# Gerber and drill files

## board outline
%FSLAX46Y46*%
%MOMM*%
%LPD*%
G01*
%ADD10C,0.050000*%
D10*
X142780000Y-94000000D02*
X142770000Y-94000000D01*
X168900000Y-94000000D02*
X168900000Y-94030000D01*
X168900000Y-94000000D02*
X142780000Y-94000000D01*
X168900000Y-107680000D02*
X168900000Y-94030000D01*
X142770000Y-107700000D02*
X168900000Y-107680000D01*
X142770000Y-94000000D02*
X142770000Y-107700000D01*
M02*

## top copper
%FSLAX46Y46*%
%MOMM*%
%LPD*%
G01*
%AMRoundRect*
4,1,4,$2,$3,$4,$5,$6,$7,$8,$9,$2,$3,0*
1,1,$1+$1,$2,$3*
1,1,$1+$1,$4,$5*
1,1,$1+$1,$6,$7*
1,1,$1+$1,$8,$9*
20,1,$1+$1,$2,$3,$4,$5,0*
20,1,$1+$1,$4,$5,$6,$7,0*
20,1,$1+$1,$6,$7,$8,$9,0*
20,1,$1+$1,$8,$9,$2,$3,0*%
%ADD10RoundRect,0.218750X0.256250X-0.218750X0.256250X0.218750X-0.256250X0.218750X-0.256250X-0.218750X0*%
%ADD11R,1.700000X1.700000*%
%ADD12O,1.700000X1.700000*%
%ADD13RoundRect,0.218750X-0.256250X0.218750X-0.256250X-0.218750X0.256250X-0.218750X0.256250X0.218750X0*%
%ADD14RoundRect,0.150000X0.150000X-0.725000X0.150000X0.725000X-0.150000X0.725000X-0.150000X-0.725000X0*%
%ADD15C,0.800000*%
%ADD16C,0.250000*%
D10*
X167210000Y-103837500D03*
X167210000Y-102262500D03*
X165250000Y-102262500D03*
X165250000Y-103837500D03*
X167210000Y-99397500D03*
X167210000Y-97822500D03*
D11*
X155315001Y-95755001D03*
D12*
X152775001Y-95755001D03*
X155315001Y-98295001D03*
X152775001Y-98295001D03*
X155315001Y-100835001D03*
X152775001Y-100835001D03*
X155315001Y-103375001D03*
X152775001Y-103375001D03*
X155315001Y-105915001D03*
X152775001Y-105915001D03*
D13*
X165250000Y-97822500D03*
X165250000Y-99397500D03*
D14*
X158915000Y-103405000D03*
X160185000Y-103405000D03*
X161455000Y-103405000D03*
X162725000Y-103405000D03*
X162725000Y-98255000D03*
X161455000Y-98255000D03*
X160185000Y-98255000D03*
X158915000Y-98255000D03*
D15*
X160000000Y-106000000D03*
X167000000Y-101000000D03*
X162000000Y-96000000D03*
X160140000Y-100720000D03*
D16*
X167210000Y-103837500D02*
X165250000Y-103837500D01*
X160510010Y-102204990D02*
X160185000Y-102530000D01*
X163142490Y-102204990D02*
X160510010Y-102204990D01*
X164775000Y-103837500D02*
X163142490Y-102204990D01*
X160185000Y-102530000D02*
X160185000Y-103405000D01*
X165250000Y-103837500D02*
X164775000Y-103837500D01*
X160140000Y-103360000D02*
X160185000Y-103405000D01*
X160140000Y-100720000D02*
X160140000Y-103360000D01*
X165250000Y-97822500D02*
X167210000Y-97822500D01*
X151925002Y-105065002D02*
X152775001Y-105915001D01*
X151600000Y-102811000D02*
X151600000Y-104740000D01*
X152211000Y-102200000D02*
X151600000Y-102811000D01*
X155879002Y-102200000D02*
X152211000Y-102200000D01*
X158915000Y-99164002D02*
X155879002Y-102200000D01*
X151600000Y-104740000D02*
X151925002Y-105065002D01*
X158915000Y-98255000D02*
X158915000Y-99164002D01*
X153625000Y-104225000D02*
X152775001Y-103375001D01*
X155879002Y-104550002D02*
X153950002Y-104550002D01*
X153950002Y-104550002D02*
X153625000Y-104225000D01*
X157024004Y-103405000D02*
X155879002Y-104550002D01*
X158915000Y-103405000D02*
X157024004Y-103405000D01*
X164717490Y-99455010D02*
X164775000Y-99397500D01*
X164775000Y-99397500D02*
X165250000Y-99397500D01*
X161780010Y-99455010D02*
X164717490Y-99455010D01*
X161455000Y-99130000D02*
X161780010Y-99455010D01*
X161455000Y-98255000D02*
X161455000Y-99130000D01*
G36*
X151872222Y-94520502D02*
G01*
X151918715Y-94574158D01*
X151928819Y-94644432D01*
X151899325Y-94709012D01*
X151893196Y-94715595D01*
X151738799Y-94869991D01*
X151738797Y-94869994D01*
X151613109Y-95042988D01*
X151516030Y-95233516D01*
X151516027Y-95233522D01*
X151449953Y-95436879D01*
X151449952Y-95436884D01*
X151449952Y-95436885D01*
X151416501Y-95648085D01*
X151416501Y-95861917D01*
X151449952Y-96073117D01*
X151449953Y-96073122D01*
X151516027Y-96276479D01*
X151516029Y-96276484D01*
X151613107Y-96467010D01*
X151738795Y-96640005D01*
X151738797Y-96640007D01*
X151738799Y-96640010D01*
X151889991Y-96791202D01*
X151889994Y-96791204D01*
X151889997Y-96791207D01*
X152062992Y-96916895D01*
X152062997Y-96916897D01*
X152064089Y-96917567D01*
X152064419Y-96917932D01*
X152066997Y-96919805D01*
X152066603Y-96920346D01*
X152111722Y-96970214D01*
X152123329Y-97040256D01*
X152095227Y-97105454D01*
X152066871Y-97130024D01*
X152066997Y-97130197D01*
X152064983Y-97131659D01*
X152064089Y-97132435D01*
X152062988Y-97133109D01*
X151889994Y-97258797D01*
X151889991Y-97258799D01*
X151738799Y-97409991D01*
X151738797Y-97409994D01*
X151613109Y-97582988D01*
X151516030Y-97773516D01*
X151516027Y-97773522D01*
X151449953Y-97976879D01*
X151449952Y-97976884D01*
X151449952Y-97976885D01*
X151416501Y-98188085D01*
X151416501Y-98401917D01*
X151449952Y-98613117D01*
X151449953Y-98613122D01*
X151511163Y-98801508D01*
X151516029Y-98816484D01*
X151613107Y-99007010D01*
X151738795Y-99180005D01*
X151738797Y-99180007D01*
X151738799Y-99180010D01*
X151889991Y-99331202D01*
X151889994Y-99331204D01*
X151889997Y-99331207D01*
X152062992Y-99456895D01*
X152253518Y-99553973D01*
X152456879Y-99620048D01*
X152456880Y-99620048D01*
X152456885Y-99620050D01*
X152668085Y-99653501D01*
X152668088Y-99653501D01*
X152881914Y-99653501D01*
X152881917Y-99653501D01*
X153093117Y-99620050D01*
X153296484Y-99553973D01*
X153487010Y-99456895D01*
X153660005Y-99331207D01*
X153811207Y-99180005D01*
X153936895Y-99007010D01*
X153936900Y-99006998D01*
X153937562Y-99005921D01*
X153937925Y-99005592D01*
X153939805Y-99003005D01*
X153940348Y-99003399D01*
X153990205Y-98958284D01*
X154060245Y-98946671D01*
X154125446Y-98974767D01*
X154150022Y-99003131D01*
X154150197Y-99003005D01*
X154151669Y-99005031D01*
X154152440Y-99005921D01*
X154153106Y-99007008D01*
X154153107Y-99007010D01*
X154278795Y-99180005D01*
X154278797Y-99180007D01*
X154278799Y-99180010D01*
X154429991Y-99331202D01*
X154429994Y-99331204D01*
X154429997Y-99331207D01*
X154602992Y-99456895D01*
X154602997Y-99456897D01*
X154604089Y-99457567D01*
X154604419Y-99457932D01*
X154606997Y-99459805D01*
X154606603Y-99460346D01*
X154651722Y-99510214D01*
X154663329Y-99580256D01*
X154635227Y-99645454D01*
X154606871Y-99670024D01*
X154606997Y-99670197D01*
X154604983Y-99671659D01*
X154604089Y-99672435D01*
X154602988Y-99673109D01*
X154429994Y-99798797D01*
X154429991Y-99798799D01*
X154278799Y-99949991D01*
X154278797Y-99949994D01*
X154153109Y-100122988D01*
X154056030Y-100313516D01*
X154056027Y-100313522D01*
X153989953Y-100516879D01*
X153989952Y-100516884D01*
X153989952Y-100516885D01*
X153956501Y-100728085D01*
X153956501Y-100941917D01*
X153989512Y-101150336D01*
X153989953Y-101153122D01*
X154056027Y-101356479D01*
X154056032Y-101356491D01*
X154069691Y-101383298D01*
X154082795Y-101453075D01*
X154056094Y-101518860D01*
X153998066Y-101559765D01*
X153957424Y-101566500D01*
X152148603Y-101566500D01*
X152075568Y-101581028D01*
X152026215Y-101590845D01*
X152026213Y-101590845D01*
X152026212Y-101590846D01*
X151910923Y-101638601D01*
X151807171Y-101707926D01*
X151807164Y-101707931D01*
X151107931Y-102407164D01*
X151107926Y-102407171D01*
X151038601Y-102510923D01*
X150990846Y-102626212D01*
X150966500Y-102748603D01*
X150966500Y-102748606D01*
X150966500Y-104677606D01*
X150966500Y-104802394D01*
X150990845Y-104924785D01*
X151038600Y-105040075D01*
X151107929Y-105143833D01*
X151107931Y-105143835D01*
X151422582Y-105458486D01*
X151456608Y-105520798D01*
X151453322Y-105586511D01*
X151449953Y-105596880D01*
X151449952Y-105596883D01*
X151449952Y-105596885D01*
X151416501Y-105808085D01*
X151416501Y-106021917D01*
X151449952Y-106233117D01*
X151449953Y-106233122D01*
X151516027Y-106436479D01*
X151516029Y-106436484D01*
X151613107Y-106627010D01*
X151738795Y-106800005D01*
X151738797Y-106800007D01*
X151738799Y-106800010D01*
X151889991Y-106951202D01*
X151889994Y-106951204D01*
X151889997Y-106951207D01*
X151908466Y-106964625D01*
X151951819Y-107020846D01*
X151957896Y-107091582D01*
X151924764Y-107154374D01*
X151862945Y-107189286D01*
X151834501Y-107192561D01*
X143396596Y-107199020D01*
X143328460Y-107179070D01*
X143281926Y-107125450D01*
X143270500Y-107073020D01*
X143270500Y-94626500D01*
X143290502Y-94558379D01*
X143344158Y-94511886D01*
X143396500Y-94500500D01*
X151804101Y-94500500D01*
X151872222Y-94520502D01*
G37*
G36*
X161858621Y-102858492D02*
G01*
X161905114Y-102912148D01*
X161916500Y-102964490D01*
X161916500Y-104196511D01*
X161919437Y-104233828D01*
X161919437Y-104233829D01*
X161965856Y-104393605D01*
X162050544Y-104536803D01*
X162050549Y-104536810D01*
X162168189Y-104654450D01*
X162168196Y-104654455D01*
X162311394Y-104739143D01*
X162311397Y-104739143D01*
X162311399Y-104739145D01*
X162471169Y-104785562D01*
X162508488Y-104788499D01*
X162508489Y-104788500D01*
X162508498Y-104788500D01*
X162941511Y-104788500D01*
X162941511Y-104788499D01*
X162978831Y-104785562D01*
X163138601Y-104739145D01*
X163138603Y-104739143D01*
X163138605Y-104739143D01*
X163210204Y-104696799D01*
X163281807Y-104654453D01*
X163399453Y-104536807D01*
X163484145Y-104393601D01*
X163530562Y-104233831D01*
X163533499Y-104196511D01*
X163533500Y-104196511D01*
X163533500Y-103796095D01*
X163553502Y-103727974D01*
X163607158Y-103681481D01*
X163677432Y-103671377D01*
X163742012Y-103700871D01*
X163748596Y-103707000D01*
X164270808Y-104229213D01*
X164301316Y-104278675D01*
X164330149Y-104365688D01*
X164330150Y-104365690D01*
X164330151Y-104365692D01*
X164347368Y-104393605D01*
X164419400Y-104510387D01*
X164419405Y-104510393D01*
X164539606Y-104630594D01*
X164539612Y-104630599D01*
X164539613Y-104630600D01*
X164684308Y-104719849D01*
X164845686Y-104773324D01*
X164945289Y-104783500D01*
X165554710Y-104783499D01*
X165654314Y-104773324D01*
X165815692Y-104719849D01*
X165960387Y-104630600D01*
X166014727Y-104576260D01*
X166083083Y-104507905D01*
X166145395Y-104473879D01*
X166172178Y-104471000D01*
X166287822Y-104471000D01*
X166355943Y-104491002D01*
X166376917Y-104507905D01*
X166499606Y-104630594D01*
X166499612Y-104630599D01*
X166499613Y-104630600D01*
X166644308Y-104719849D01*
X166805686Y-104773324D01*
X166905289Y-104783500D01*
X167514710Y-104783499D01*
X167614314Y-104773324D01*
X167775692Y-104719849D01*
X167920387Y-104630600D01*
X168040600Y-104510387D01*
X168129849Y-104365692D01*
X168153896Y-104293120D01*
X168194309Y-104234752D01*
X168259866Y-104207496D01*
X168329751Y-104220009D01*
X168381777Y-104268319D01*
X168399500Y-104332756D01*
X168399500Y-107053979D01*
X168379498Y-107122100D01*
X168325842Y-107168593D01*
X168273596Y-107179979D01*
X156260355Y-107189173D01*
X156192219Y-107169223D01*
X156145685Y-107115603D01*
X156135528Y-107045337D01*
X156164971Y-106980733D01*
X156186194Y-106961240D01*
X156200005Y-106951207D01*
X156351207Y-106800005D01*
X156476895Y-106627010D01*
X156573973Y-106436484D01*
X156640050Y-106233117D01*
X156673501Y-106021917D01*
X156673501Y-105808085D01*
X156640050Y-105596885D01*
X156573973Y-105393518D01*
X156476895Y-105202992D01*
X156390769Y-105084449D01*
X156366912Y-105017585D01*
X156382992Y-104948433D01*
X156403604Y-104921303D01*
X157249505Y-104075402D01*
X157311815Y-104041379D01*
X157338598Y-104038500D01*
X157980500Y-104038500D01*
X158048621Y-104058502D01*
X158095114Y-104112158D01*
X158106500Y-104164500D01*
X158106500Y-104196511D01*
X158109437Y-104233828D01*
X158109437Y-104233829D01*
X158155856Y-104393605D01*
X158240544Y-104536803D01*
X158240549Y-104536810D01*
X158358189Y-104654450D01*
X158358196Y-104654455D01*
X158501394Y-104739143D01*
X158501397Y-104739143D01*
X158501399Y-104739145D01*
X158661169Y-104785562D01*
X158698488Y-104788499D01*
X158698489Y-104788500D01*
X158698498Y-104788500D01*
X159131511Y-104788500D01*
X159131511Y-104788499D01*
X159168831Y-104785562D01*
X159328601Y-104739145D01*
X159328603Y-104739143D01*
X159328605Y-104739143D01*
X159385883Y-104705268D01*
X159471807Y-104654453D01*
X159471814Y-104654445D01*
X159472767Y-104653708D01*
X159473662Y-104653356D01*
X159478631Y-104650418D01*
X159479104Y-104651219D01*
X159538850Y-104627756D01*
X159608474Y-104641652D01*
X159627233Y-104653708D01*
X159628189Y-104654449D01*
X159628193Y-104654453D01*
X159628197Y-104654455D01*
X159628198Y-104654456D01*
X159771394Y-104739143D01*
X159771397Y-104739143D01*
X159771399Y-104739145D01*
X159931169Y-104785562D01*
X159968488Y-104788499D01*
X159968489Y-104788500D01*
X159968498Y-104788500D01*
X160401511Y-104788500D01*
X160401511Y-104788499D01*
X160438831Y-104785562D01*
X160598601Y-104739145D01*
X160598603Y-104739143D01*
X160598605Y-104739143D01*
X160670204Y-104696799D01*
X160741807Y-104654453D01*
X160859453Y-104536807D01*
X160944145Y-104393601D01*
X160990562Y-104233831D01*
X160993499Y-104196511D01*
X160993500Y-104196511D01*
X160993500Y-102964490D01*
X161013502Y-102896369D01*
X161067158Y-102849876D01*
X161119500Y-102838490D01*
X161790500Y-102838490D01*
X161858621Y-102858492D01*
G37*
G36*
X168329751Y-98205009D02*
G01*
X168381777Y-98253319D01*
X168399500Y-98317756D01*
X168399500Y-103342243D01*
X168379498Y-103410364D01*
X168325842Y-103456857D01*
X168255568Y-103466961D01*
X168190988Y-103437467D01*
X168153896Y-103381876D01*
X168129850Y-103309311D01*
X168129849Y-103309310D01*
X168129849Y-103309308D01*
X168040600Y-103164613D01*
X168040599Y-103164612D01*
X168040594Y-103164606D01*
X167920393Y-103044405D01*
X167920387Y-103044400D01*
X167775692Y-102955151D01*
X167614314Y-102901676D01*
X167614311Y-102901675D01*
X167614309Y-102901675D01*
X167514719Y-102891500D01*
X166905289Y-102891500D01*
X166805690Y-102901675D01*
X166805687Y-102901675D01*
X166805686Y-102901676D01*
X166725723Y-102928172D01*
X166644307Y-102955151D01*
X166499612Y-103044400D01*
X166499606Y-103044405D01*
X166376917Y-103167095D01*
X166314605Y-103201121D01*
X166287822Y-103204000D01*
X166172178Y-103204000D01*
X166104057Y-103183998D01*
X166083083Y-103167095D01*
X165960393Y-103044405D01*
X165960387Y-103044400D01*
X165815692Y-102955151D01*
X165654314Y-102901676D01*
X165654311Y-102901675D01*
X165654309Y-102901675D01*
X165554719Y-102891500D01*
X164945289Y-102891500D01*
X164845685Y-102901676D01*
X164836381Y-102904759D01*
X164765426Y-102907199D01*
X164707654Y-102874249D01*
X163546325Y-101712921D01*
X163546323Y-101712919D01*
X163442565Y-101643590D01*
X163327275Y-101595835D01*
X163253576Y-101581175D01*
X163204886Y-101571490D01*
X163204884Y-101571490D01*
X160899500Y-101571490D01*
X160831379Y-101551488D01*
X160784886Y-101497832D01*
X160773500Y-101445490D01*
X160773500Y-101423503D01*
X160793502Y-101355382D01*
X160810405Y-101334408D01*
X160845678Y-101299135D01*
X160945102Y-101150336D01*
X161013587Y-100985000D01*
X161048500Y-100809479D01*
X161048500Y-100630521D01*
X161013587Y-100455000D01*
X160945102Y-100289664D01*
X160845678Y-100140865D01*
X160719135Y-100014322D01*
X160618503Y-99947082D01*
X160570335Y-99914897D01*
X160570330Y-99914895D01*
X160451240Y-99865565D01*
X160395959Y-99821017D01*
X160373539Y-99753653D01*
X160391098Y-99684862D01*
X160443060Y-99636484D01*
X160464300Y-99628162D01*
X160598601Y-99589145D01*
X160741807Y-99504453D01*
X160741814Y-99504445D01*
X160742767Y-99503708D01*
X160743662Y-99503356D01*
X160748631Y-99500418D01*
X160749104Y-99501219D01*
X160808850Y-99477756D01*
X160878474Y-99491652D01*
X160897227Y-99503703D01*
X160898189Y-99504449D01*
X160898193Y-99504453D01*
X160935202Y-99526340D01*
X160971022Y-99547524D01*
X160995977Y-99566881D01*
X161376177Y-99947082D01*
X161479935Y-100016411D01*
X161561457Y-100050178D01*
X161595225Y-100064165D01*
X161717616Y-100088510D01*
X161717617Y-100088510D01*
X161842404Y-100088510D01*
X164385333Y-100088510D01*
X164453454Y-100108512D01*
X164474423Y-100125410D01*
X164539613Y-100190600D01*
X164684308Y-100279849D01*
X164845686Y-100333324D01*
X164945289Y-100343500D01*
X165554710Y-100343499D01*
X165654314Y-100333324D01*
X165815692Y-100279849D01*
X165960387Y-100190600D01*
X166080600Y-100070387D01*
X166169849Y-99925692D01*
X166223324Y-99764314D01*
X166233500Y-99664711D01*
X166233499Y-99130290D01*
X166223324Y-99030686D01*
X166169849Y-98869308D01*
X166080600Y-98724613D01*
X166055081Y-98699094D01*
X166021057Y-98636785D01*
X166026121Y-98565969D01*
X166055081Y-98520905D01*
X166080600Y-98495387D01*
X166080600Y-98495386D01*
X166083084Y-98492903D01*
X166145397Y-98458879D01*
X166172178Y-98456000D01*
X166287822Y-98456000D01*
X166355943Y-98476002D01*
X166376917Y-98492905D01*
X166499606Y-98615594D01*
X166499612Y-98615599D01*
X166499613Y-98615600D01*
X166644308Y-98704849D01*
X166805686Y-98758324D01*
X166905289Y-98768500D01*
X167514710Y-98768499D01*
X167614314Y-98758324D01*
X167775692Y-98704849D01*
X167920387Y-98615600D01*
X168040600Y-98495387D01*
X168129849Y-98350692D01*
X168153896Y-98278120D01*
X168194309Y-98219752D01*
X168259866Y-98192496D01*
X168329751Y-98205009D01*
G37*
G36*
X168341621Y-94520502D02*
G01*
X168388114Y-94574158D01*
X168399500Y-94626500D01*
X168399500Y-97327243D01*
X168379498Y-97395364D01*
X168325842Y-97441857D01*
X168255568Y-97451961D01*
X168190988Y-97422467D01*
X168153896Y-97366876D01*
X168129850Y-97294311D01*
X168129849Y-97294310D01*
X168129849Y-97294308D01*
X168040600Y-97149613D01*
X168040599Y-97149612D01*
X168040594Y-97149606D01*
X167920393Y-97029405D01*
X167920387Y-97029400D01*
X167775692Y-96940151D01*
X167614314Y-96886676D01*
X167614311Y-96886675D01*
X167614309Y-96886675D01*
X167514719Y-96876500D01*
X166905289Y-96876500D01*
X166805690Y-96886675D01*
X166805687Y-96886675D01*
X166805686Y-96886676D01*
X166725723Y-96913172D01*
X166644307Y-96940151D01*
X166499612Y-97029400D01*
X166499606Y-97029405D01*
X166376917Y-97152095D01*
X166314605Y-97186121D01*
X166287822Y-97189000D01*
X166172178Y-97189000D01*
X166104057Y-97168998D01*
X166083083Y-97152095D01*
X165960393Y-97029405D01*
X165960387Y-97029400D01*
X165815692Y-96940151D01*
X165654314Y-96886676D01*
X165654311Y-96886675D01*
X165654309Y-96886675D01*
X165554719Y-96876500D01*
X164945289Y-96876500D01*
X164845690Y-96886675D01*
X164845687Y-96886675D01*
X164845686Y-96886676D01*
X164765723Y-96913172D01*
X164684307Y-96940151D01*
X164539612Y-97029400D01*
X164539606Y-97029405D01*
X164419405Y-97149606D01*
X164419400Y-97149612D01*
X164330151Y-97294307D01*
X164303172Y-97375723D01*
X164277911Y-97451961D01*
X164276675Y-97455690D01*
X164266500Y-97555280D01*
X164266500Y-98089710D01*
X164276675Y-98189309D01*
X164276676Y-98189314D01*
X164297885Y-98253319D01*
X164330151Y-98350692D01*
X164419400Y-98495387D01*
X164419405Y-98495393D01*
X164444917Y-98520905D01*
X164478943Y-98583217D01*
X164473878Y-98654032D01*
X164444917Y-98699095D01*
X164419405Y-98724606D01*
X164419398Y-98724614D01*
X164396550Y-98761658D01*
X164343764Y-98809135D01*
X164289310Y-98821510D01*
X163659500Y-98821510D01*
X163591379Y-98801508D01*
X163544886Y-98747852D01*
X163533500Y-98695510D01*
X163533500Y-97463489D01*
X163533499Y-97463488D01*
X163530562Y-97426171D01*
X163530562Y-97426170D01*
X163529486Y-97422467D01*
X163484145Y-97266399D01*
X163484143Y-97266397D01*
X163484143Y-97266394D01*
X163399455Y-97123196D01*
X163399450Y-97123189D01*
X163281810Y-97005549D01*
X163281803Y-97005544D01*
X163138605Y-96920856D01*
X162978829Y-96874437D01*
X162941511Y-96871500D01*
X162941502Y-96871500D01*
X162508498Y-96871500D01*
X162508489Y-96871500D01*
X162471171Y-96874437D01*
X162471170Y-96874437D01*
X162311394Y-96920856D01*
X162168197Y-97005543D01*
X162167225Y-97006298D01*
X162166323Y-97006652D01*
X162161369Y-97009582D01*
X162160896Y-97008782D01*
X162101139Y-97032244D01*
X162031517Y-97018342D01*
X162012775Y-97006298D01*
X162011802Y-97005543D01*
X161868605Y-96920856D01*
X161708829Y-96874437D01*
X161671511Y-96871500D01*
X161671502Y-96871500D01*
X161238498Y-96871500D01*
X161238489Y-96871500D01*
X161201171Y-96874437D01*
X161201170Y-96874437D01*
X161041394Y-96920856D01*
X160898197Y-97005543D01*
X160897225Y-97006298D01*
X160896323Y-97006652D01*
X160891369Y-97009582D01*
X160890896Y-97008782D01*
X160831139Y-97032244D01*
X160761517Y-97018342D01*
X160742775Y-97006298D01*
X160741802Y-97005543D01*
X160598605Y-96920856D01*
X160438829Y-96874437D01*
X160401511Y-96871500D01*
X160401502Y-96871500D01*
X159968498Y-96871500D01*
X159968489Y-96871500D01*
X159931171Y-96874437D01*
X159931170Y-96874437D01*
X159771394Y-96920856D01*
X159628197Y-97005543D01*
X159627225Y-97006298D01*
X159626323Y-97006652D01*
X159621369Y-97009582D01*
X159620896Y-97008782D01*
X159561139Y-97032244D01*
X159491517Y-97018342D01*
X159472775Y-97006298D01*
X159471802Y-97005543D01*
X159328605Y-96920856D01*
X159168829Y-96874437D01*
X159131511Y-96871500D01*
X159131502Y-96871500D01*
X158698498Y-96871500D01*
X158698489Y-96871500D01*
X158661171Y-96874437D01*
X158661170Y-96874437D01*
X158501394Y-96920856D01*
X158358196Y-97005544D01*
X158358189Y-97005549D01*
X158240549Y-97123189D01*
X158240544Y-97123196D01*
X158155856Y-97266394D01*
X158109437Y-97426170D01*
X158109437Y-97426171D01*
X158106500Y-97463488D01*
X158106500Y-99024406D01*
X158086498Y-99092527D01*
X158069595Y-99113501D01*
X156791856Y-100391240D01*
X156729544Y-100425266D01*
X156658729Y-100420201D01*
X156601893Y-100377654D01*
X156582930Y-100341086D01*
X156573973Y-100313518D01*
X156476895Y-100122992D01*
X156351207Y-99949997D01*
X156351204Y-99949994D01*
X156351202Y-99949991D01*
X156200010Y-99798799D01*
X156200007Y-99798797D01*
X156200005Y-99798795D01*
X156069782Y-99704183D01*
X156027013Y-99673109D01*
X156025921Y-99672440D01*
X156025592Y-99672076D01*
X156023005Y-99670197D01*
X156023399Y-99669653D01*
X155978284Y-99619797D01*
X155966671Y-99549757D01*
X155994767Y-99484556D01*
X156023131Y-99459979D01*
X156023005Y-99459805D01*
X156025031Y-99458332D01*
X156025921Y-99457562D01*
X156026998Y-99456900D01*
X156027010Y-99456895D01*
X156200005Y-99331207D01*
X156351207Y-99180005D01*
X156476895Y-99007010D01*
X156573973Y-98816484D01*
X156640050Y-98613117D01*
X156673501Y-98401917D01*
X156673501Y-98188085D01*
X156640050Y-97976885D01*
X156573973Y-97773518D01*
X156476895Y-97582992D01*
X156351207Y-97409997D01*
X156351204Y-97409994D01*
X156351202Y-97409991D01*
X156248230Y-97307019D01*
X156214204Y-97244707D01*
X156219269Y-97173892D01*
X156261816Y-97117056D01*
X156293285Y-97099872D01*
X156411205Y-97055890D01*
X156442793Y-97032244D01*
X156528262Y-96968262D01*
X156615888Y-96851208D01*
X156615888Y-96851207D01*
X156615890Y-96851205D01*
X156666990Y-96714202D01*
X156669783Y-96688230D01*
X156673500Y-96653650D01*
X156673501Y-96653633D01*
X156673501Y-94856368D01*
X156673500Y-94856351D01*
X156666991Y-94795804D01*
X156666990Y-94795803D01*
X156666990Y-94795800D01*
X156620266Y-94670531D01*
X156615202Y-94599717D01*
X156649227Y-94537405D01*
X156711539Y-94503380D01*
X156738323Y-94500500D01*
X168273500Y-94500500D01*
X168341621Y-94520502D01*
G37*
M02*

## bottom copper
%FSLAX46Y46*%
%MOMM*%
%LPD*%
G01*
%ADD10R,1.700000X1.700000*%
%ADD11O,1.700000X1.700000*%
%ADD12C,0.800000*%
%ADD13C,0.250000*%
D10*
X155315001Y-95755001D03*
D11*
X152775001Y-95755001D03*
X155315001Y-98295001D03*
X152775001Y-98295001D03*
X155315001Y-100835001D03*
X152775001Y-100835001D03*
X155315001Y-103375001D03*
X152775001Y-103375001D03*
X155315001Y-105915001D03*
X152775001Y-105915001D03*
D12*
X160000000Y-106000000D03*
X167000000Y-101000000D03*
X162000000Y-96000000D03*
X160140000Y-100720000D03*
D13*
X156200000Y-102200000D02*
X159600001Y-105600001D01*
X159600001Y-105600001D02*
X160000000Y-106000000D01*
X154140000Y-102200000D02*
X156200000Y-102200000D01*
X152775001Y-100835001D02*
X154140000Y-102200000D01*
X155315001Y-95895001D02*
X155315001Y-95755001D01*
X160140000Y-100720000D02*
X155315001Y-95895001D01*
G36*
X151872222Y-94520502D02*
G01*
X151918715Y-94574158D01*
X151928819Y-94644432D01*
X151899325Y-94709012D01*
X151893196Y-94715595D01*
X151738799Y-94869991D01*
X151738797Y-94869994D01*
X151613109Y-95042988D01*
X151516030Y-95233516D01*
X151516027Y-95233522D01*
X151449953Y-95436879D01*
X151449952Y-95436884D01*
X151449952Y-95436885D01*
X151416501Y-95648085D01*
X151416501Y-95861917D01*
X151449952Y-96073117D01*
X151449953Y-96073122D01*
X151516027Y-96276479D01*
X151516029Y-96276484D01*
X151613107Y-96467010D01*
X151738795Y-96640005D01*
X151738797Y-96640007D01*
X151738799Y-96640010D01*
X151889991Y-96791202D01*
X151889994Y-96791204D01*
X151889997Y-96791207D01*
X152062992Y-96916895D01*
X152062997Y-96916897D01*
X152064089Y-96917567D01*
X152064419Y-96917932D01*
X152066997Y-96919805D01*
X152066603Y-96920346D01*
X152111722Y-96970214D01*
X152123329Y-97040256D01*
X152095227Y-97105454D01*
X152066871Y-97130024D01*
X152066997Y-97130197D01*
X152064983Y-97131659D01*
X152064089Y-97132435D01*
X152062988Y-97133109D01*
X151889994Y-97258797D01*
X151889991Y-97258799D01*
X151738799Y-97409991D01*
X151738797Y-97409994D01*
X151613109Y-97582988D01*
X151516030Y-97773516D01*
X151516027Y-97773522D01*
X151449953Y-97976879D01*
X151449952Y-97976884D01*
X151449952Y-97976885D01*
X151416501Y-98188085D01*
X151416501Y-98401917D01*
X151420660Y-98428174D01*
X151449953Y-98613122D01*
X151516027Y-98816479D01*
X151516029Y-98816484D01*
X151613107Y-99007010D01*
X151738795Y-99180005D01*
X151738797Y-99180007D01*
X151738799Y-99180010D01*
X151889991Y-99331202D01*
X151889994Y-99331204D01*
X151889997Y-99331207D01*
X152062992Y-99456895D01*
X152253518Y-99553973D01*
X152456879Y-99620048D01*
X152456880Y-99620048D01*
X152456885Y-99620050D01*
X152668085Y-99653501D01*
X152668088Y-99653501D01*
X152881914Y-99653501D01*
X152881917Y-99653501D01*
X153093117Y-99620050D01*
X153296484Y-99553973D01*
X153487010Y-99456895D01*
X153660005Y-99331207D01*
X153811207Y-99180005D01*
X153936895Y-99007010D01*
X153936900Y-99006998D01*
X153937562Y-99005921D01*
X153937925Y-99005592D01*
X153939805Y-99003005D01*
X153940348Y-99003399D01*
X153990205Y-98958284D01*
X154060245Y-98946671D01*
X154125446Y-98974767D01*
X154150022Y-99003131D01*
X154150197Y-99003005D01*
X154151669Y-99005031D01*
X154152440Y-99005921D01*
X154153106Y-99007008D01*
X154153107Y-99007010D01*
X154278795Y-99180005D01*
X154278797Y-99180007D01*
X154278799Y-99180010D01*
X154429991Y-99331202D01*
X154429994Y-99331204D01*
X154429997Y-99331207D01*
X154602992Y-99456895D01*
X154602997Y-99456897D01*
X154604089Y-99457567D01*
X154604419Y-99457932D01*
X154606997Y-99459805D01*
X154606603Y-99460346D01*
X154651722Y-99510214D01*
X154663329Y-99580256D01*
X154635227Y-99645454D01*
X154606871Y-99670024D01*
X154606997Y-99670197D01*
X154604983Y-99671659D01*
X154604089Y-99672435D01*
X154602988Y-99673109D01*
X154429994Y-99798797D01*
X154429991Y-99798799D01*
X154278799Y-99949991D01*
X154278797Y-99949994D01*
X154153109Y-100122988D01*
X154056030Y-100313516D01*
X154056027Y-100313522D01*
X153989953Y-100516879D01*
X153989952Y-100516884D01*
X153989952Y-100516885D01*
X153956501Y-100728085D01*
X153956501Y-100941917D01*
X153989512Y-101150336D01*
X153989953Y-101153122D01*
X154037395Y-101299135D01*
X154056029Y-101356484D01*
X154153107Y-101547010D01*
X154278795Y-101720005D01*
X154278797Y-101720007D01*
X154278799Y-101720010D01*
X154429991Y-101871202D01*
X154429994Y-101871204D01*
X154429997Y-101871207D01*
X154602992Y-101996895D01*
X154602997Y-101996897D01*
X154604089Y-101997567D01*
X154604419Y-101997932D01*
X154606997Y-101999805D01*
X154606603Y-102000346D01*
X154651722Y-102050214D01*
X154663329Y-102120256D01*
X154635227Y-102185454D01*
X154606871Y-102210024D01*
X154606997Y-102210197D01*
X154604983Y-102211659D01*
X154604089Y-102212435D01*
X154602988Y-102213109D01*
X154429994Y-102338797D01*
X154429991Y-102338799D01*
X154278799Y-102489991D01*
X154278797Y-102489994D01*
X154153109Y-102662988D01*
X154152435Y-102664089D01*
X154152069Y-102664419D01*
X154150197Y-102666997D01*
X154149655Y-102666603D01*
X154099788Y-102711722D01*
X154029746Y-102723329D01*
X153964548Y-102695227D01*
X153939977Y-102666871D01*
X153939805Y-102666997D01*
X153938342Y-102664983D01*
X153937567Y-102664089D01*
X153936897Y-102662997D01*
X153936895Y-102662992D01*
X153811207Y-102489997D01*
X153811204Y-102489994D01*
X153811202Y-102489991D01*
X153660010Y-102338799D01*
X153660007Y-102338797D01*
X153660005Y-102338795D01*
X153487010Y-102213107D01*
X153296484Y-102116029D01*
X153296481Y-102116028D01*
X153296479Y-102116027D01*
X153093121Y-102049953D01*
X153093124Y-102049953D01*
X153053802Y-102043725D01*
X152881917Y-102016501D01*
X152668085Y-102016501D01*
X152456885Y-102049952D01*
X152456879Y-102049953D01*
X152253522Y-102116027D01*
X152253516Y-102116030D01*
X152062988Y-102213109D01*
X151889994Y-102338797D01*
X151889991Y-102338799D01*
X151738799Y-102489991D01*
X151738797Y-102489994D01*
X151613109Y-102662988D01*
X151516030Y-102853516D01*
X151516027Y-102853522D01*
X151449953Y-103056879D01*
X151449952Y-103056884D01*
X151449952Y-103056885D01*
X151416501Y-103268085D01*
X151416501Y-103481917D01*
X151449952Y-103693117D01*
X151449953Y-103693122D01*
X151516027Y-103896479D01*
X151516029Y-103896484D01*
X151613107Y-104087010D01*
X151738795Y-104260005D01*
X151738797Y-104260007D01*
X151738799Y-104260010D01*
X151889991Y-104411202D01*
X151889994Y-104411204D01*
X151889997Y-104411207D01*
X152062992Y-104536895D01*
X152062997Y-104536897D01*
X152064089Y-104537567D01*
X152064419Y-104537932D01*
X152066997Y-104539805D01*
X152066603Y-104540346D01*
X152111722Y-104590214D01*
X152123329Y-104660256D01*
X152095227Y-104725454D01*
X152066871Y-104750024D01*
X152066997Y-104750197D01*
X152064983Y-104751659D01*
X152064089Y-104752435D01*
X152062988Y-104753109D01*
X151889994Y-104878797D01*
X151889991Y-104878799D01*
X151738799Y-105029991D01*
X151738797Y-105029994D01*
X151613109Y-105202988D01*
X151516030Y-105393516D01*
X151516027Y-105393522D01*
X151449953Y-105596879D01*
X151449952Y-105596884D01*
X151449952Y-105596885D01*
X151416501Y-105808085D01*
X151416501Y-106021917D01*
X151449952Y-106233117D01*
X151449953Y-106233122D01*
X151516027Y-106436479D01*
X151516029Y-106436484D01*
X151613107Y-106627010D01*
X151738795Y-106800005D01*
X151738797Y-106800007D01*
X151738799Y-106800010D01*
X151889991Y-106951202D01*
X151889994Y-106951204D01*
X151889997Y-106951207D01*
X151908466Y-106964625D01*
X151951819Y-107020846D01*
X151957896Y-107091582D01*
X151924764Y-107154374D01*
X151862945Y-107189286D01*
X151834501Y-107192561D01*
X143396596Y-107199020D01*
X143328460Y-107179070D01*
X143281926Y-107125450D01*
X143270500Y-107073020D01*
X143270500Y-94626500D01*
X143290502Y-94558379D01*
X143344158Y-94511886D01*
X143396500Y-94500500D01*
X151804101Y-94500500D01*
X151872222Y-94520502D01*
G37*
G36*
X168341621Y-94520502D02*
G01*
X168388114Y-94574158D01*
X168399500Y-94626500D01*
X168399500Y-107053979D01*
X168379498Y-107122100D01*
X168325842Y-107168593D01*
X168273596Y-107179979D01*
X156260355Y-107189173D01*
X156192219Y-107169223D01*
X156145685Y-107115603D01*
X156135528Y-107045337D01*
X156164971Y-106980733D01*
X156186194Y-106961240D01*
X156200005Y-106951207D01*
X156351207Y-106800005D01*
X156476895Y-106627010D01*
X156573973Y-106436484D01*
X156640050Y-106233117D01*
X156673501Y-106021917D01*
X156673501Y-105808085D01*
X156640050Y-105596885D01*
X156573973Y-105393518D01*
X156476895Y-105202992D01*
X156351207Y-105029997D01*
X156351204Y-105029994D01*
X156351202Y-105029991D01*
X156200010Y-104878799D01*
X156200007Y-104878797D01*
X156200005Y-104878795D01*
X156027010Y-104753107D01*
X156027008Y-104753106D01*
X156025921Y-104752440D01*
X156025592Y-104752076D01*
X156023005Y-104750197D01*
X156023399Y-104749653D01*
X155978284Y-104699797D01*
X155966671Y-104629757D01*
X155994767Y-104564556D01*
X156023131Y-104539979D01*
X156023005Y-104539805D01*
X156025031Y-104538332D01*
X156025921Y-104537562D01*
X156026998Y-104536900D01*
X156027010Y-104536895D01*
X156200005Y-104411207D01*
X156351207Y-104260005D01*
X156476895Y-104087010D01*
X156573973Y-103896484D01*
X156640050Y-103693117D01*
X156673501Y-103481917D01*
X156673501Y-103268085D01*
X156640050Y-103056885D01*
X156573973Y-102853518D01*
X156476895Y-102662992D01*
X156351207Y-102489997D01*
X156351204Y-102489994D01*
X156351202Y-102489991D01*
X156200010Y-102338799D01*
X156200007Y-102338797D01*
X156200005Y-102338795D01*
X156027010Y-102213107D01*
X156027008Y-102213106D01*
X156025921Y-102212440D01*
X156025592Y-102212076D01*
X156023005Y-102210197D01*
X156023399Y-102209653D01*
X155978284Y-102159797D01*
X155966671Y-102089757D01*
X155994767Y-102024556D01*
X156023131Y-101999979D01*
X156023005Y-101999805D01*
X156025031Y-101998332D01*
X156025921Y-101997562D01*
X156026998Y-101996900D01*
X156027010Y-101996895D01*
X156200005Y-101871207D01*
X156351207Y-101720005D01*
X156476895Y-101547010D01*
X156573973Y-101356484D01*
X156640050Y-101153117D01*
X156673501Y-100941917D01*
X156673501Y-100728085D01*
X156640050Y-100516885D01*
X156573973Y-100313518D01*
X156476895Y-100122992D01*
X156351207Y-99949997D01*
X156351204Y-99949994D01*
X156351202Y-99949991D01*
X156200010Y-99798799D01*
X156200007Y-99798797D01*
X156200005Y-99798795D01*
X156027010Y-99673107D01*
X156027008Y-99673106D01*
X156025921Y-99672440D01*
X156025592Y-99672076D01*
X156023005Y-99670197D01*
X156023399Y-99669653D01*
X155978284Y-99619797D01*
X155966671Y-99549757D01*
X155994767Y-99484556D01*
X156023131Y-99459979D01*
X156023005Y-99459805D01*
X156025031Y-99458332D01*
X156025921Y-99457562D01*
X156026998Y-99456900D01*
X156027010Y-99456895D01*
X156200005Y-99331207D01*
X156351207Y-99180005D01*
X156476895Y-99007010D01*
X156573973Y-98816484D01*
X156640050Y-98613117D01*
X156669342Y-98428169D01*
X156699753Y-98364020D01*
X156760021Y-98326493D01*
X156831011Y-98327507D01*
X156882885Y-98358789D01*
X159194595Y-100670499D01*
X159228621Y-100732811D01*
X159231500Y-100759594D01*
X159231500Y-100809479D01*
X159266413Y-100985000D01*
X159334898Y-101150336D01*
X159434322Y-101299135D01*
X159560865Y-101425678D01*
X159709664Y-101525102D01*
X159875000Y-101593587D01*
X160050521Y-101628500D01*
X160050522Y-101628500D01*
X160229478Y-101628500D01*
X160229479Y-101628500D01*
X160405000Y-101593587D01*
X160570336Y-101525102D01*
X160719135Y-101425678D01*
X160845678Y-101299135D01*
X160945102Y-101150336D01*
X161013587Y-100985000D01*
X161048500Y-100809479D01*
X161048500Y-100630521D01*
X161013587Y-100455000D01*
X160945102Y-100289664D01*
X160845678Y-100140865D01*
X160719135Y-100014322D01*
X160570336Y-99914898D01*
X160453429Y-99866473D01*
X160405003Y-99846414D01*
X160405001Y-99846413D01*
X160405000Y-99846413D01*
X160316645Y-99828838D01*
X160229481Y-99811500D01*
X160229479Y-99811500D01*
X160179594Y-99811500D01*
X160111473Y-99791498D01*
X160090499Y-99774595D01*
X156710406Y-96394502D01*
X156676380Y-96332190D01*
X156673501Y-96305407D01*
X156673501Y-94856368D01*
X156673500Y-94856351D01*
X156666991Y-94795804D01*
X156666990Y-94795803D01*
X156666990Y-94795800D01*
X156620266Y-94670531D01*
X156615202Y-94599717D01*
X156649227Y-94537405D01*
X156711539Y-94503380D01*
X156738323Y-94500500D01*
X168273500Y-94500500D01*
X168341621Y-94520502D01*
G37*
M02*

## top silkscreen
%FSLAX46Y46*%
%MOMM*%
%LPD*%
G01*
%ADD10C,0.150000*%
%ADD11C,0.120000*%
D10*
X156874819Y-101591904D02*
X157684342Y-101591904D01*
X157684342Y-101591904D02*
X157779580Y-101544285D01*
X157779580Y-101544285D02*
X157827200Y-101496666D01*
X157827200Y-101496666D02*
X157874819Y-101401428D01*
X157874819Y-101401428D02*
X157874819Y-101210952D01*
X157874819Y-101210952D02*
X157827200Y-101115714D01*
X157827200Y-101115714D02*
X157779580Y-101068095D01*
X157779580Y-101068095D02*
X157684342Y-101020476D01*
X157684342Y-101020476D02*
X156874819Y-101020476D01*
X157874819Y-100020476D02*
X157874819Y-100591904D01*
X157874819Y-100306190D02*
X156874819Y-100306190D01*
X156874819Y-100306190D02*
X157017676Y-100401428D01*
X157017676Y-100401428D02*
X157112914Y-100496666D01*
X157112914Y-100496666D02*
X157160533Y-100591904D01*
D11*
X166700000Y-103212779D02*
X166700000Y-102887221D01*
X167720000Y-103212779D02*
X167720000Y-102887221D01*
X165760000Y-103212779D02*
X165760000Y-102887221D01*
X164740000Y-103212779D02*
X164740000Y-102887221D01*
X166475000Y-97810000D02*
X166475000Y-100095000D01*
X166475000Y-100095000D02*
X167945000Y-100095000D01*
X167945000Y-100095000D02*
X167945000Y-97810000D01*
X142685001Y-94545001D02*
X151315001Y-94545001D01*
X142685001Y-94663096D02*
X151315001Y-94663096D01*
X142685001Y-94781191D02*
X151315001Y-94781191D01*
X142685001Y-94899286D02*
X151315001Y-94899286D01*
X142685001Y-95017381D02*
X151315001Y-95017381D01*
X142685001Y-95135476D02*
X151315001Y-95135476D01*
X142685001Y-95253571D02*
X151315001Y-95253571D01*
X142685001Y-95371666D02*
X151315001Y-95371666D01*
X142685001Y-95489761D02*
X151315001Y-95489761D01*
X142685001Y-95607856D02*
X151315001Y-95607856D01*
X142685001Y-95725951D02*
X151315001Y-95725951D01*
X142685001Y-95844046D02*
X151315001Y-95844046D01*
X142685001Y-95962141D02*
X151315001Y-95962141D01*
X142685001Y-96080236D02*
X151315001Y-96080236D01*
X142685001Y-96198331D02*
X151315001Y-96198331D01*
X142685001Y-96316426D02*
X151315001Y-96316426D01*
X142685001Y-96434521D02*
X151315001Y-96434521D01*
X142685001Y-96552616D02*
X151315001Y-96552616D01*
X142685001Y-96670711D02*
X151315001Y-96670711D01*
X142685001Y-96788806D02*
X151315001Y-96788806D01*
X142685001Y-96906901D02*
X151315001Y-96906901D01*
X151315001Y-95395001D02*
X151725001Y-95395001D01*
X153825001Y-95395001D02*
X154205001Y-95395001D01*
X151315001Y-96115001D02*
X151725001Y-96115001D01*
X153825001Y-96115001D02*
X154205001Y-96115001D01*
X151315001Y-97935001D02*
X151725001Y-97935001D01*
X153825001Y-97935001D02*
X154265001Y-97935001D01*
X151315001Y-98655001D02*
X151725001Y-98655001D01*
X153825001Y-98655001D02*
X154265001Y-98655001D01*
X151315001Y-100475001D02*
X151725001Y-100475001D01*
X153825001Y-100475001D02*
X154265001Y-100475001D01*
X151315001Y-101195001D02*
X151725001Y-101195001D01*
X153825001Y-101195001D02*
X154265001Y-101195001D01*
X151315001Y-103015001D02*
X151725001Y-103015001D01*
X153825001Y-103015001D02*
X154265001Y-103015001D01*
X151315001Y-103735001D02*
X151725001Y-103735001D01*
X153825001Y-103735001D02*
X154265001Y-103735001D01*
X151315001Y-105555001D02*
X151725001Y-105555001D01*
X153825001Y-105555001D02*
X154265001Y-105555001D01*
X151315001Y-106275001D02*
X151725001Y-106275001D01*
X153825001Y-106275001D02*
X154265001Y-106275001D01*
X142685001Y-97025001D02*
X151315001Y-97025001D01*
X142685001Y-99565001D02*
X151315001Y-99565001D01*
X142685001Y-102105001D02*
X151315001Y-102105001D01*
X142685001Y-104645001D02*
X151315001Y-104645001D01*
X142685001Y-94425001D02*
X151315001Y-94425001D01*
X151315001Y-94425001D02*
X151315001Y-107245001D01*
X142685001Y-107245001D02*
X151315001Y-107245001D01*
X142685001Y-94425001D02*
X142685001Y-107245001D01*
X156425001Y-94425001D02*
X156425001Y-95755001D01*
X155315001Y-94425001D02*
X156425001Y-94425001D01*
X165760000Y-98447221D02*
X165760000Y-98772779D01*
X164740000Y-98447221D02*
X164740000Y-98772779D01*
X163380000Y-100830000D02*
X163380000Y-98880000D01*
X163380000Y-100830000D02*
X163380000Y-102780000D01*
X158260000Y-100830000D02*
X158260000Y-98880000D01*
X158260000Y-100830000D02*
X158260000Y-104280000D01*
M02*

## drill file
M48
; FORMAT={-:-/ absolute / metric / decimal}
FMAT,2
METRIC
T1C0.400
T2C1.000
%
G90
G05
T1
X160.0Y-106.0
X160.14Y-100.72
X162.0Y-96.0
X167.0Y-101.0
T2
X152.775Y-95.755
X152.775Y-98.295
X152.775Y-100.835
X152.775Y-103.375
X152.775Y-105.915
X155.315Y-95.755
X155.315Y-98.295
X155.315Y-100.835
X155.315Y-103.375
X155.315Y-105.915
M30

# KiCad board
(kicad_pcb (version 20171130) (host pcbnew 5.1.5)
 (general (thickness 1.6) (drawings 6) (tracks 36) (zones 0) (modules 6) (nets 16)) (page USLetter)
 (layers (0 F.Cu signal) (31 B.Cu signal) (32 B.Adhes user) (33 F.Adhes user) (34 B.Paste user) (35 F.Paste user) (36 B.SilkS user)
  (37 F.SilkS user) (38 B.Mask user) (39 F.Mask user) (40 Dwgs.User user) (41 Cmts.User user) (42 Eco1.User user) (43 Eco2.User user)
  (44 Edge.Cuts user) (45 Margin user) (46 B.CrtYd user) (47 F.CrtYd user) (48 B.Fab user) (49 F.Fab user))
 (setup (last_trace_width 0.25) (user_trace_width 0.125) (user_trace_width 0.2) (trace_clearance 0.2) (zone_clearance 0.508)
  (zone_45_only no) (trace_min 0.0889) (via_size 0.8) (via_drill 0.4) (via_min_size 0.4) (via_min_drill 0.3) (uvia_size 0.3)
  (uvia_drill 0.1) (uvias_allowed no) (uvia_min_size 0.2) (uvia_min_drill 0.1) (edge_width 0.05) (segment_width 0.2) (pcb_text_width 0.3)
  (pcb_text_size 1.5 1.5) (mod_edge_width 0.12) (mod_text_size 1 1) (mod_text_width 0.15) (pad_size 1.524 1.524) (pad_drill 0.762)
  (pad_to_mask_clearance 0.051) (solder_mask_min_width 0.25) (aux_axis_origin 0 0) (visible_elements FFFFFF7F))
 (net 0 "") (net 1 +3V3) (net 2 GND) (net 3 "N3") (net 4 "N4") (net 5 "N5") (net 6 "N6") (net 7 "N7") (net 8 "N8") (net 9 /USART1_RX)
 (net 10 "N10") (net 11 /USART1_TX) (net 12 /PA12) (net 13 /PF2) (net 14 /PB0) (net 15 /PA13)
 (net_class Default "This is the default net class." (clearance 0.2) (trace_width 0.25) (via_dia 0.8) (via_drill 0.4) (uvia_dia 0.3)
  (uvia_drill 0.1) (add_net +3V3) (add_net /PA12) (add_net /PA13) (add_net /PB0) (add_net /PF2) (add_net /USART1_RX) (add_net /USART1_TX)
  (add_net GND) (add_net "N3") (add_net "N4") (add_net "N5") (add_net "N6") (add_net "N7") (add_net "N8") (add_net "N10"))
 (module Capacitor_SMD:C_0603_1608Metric (layer F.Cu) (at 167.21 103.05 90)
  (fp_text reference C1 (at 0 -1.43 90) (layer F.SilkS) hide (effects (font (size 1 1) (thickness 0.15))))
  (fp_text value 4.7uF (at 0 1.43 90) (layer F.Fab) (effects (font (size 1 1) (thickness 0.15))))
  (fp_line (start -0.162779 -0.51) (end 0.162779 -0.51) (layer F.SilkS) (width 0.12))
  (fp_line (start -0.162779 0.51) (end 0.162779 0.51) (layer F.SilkS) (width 0.12))
  (pad 1 smd roundrect (at -0.7875 0 90) (size 0.875 0.95) (layers F.Cu F.Paste F.Mask) (roundrect_rratio 0.25) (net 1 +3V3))
  (pad 2 smd roundrect (at 0.7875 0 90) (size 0.875 0.95) (layers F.Cu F.Paste F.Mask) (roundrect_rratio 0.25) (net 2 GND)))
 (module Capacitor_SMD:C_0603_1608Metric (layer F.Cu) (at 165.25 103.05 90)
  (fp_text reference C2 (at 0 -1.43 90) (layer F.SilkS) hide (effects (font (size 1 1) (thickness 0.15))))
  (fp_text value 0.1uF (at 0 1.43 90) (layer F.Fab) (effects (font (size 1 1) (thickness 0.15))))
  (fp_line (start -0.162779 0.51) (end 0.162779 0.51) (layer F.SilkS) (width 0.12))
  (fp_line (start -0.162779 -0.51) (end 0.162779 -0.51) (layer F.SilkS) (width 0.12))
  (pad 2 smd roundrect (at 0.7875 0 90) (size 0.875 0.95) (layers F.Cu F.Paste F.Mask) (roundrect_rratio 0.25) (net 2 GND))
  (pad 1 smd roundrect (at -0.7875 0 90) (size 0.875 0.95) (layers F.Cu F.Paste F.Mask) (roundrect_rratio 0.25) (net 1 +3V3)))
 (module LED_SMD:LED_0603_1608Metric (layer F.Cu) (at 167.21 98.61 90)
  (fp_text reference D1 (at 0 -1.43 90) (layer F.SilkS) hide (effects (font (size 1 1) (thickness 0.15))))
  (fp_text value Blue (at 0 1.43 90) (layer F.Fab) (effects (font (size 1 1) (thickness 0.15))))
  (fp_line (start 0.8 -0.735) (end -1.485 -0.735) (layer F.SilkS) (width 0.12))
  (fp_line (start -1.485 -0.735) (end -1.485 0.735) (layer F.SilkS) (width 0.12))
  (fp_line (start -1.485 0.735) (end 0.8 0.735) (layer F.SilkS) (width 0.12))
  (pad 1 smd roundrect (at -0.7875 0 90) (size 0.875 0.95) (layers F.Cu F.Paste F.Mask) (roundrect_rratio 0.25) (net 2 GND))
  (pad 2 smd roundrect (at 0.7875 0 90) (size 0.875 0.95) (layers F.Cu F.Paste F.Mask) (roundrect_rratio 0.25) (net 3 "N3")))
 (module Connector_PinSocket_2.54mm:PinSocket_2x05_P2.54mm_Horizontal (layer F.Cu) (at 155.315001 95.755001)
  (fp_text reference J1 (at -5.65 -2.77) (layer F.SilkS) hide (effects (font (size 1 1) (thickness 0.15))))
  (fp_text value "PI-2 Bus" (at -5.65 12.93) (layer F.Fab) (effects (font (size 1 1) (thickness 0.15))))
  (fp_line (start -12.63 -1.21) (end -4 -1.21) (layer F.SilkS) (width 0.12))
  (fp_line (start -12.63 -1.091905) (end -4 -1.091905) (layer F.SilkS) (width 0.12))
  (fp_line (start -12.63 -0.97381) (end -4 -0.97381) (layer F.SilkS) (width 0.12))
  (fp_line (start -12.63 -0.855715) (end -4 -0.855715) (layer F.SilkS) (width 0.12))
  (fp_line (start -12.63 -0.73762) (end -4 -0.73762) (layer F.SilkS) (width 0.12))
  (fp_line (start -12.63 -0.619525) (end -4 -0.619525) (layer F.SilkS) (width 0.12))
  (fp_line (start -12.63 -0.50143) (end -4 -0.50143) (layer F.SilkS) (width 0.12))
  (fp_line (start -12.63 -0.383335) (end -4 -0.383335) (layer F.SilkS) (width 0.12))
  (fp_line (start -12.63 -0.26524) (end -4 -0.26524) (layer F.SilkS) (width 0.12))
  (fp_line (start -12.63 -0.147145) (end -4 -0.147145) (layer F.SilkS) (width 0.12))
  (fp_line (start -12.63 -0.02905) (end -4 -0.02905) (layer F.SilkS) (width 0.12))
  (fp_line (start -12.63 0.089045) (end -4 0.089045) (layer F.SilkS) (width 0.12))
  (fp_line (start -12.63 0.20714) (end -4 0.20714) (layer F.SilkS) (width 0.12))
  (fp_line (start -12.63 0.325235) (end -4 0.325235) (layer F.SilkS) (width 0.12))
  (fp_line (start -12.63 0.44333) (end -4 0.44333) (layer F.SilkS) (width 0.12))
  (fp_line (start -12.63 0.561425) (end -4 0.561425) (layer F.SilkS) (width 0.12))
  (fp_line (start -12.63 0.67952) (end -4 0.67952) (layer F.SilkS) (width 0.12))
  (fp_line (start -12.63 0.797615) (end -4 0.797615) (layer F.SilkS) (width 0.12))
  (fp_line (start -12.63 0.91571) (end -4 0.91571) (layer F.SilkS) (width 0.12))
  (fp_line (start -12.63 1.033805) (end -4 1.033805) (layer F.SilkS) (width 0.12))
  (fp_line (start -12.63 1.1519) (end -4 1.1519) (layer F.SilkS) (width 0.12))
  (fp_line (start -4 -0.36) (end -3.59 -0.36) (layer F.SilkS) (width 0.12))
  (fp_line (start -1.49 -0.36) (end -1.11 -0.36) (layer F.SilkS) (width 0.12))
  (fp_line (start -4 0.36) (end -3.59 0.36) (layer F.SilkS) (width 0.12))
  (fp_line (start -1.49 0.36) (end -1.11 0.36) (layer F.SilkS) (width 0.12))
  (fp_line (start -4 2.18) (end -3.59 2.18) (layer F.SilkS) (width 0.12))
  (fp_line (start -1.49 2.18) (end -1.05 2.18) (layer F.SilkS) (width 0.12))
  (fp_line (start -4 2.9) (end -3.59 2.9) (layer F.SilkS) (width 0.12))
  (fp_line (start -1.49 2.9) (end -1.05 2.9) (layer F.SilkS) (width 0.12))
  (fp_line (start -4 4.72) (end -3.59 4.72) (layer F.SilkS) (width 0.12))
  (fp_line (start -1.49 4.72) (end -1.05 4.72) (layer F.SilkS) (width 0.12))
  (fp_line (start -4 5.44) (end -3.59 5.44) (layer F.SilkS) (width 0.12))
  (fp_line (start -1.49 5.44) (end -1.05 5.44) (layer F.SilkS) (width 0.12))
  (fp_line (start -4 7.26) (end -3.59 7.26) (layer F.SilkS) (width 0.12))
  (fp_line (start -1.49 7.26) (end -1.05 7.26) (layer F.SilkS) (width 0.12))
  (fp_line (start -4 7.98) (end -3.59 7.98) (layer F.SilkS) (width 0.12))
  (fp_line (start -1.49 7.98) (end -1.05 7.98) (layer F.SilkS) (width 0.12))
  (fp_line (start -4 9.8) (end -3.59 9.8) (layer F.SilkS) (width 0.12))
  (fp_line (start -1.49 9.8) (end -1.05 9.8) (layer F.SilkS) (width 0.12))
  (fp_line (start -4 10.52) (end -3.59 10.52) (layer F.SilkS) (width 0.12))
  (fp_line (start -1.49 10.52) (end -1.05 10.52) (layer F.SilkS) (width 0.12))
  (fp_line (start -12.63 1.27) (end -4 1.27) (layer F.SilkS) (width 0.12))
  (fp_line (start -12.63 3.81) (end -4 3.81) (layer F.SilkS) (width 0.12))
  (fp_line (start -12.63 6.35) (end -4 6.35) (layer F.SilkS) (width 0.12))
  (fp_line (start -12.63 8.89) (end -4 8.89) (layer F.SilkS) (width 0.12))
  (fp_line (start -12.63 -1.33) (end -4 -1.33) (layer F.SilkS) (width 0.12))
  (fp_line (start -4 -1.33) (end -4 11.49) (layer F.SilkS) (width 0.12))
  (fp_line (start -12.63 11.49) (end -4 11.49) (layer F.SilkS) (width 0.12))
  (fp_line (start -12.63 -1.33) (end -12.63 11.49) (layer F.SilkS) (width 0.12))
  (fp_line (start 1.11 -1.33) (end 1.11 0) (layer F.SilkS) (width 0.12))
  (fp_line (start 0 -1.33) (end 1.11 -1.33) (layer F.SilkS) (width 0.12))
  (pad 1 thru_hole rect (at 0 0) (size 1.7 1.7) (drill 1) (layers *.Cu *.Mask) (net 1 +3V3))
  (pad 2 thru_hole oval (at -2.54 0) (size 1.7 1.7) (drill 1) (layers *.Cu *.Mask) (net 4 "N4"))
  (pad 3 thru_hole oval (at 0 2.54) (size 1.7 1.7) (drill 1) (layers *.Cu *.Mask) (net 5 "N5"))
  (pad 4 thru_hole oval (at -2.54 2.54) (size 1.7 1.7) (drill 1) (layers *.Cu *.Mask) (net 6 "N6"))
  (pad 5 thru_hole oval (at 0 5.08) (size 1.7 1.7) (drill 1) (layers *.Cu *.Mask) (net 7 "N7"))
  (pad 6 thru_hole oval (at -2.54 5.08) (size 1.7 1.7) (drill 1) (layers *.Cu *.Mask) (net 2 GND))
  (pad 7 thru_hole oval (at 0 7.62) (size 1.7 1.7) (drill 1) (layers *.Cu *.Mask) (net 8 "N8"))
  (pad 8 thru_hole oval (at -2.54 7.62) (size 1.7 1.7) (drill 1) (layers *.Cu *.Mask) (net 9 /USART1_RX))
  (pad 9 thru_hole oval (at 0 10.16) (size 1.7 1.7) (drill 1) (layers *.Cu *.Mask) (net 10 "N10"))
  (pad 10 thru_hole oval (at -2.54 10.16) (size 1.7 1.7) (drill 1) (layers *.Cu *.Mask) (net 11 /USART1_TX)))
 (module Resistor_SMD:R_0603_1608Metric (layer F.Cu) (at 165.25 98.61 270)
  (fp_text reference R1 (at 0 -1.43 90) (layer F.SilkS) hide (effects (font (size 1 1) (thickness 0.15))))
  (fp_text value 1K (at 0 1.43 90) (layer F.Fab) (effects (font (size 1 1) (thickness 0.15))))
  (fp_line (start -0.162779 -0.51) (end 0.162779 -0.51) (layer F.SilkS) (width 0.12))
  (fp_line (start -0.162779 0.51) (end 0.162779 0.51) (layer F.SilkS) (width 0.12))
  (pad 1 smd roundrect (at -0.7875 0 270) (size 0.875 0.95) (layers F.Cu F.Paste F.Mask) (roundrect_rratio 0.25) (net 3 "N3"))
  (pad 2 smd roundrect (at 0.7875 0 270) (size 0.875 0.95) (layers F.Cu F.Paste F.Mask) (roundrect_rratio 0.25) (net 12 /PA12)))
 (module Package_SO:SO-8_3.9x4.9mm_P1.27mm (layer F.Cu) (at 160.82 100.83 90)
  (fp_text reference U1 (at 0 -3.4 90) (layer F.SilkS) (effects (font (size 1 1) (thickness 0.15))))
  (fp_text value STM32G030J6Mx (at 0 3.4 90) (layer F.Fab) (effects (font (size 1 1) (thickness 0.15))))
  (fp_line (start 0 2.56) (end 1.95 2.56) (layer F.SilkS) (width 0.12))
  (fp_line (start 0 2.56) (end -1.95 2.56) (layer F.SilkS) (width 0.12))
  (fp_line (start 0 -2.56) (end 1.95 -2.56) (layer F.SilkS) (width 0.12))
  (fp_line (start 0 -2.56) (end -3.45 -2.56) (layer F.SilkS) (width 0.12))
  (pad 1 smd roundrect (at -2.575 -1.905 90) (size 1.75 0.6) (layers F.Cu F.Paste F.Mask) (roundrect_rratio 0.25) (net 9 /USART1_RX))
  (pad 2 smd roundrect (at -2.575 -0.635 90) (size 1.75 0.6) (layers F.Cu F.Paste F.Mask) (roundrect_rratio 0.25) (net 1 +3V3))
  (pad 3 smd roundrect (at -2.575 0.635 90) (size 1.75 0.6) (layers F.Cu F.Paste F.Mask) (roundrect_rratio 0.25) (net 2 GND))
  (pad 4 smd roundrect (at -2.575 1.905 90) (size 1.75 0.6) (layers F.Cu F.Paste F.Mask) (roundrect_rratio 0.25) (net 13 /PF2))
  (pad 5 smd roundrect (at 2.575 1.905 90) (size 1.75 0.6) (layers F.Cu F.Paste F.Mask) (roundrect_rratio 0.25) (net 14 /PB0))
  (pad 6 smd roundrect (at 2.575 0.635 90) (size 1.75 0.6) (layers F.Cu F.Paste F.Mask) (roundrect_rratio 0.25) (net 12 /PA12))
  (pad 7 smd roundrect (at 2.575 -0.635 90) (size 1.75 0.6) (layers F.Cu F.Paste F.Mask) (roundrect_rratio 0.25) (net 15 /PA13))
  (pad 8 smd roundrect (at 2.575 -1.905 90) (size 1.75 0.6) (layers F.Cu F.Paste F.Mask) (roundrect_rratio 0.25) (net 11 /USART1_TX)))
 (gr_line (start 142.78 94) (end 142.77 94) (layer Edge.Cuts) (width 0.05))
 (gr_line (start 168.9 94) (end 168.9 94.03) (layer Edge.Cuts) (width 0.05))
 (gr_line (start 168.9 94) (end 142.78 94) (layer Edge.Cuts) (width 0.05))
 (gr_line (start 168.9 107.68) (end 168.9 94.03) (layer Edge.Cuts) (width 0.05))
 (gr_line (start 142.77 107.7) (end 168.9 107.68) (layer Edge.Cuts) (width 0.05))
 (gr_line (start 142.77 94) (end 142.77 107.7) (layer Edge.Cuts) (width 0.05))
 (via (at 160 106) (size 0.8) (drill 0.4) (layers F.Cu B.Cu) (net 2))
 (via (at 167 101) (size 0.8) (drill 0.4) (layers F.Cu B.Cu) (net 2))
 (segment (start 156.2 102.2) (end 159.600001 105.600001) (width 0.25) (layer B.Cu) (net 2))
 (segment (start 159.600001 105.600001) (end 160 106) (width 0.25) (layer B.Cu) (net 2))
 (segment (start 154.14 102.2) (end 156.2 102.2) (width 0.25) (layer B.Cu) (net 2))
 (segment (start 152.775001 100.835001) (end 154.14 102.2) (width 0.25) (layer B.Cu) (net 2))
 (via (at 162 96) (size 0.8) (drill 0.4) (layers F.Cu B.Cu) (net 2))
 (via (at 160.14 100.72) (size 0.8) (drill 0.4) (layers F.Cu B.Cu) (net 1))
 (segment (start 167.21 103.8375) (end 165.25 103.8375) (width 0.25) (layer F.Cu) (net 1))
 (segment (start 160.51001 102.20499) (end 160.185 102.53) (width 0.25) (layer F.Cu) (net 1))
 (segment (start 163.14249 102.20499) (end 160.51001 102.20499) (width 0.25) (layer F.Cu) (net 1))
 (segment (start 164.775 103.8375) (end 163.14249 102.20499) (width 0.25) (layer F.Cu) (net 1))
 (segment (start 160.185 102.53) (end 160.185 103.405) (width 0.25) (layer F.Cu) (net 1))
 (segment (start 165.25 103.8375) (end 164.775 103.8375) (width 0.25) (layer F.Cu) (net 1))
 (segment (start 160.14 103.36) (end 160.185 103.405) (width 0.25) (layer F.Cu) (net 1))
 (segment (start 160.14 100.72) (end 160.14 103.36) (width 0.25) (layer F.Cu) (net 1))
 (segment (start 155.315001 95.895001) (end 155.315001 95.755001) (width 0.25) (layer B.Cu) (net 1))
 (segment (start 160.14 100.72) (end 155.315001 95.895001) (width 0.25) (layer B.Cu) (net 1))
 (segment (start 165.25 97.8225) (end 167.21 97.8225) (width 0.25) (layer F.Cu) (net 3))
 (segment (start 151.925002 105.065002) (end 152.775001 105.915001) (width 0.25) (layer F.Cu) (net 11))
 (segment (start 151.6 102.811) (end 151.6 104.74) (width 0.25) (layer F.Cu) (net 11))
 (segment (start 152.211 102.2) (end 151.6 102.811) (width 0.25) (layer F.Cu) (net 11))
 (segment (start 155.879002 102.2) (end 152.211 102.2) (width 0.25) (layer F.Cu) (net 11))
 (segment (start 158.915 99.164002) (end 155.879002 102.2) (width 0.25) (layer F.Cu) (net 11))
 (segment (start 151.6 104.74) (end 151.925002 105.065002) (width 0.25) (layer F.Cu) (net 11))
 (segment (start 158.915 98.255) (end 158.915 99.164002) (width 0.25) (layer F.Cu) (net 11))
 (segment (start 153.625 104.225) (end 152.775001 103.375001) (width 0.25) (layer F.Cu) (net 9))
 (segment (start 155.879002 104.550002) (end 153.950002 104.550002) (width 0.25) (layer F.Cu) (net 9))
 (segment (start 153.950002 104.550002) (end 153.625 104.225) (width 0.25) (layer F.Cu) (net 9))
 (segment (start 157.024004 103.405) (end 155.879002 104.550002) (width 0.25) (layer F.Cu) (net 9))
 (segment (start 158.915 103.405) (end 157.024004 103.405) (width 0.25) (layer F.Cu) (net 9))
 (segment (start 164.71749 99.45501) (end 164.775 99.3975) (width 0.25) (layer F.Cu) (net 12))
 (segment (start 164.775 99.3975) (end 165.25 99.3975) (width 0.25) (layer F.Cu) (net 12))
 (segment (start 161.78001 99.45501) (end 164.71749 99.45501) (width 0.25) (layer F.Cu) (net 12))
 (segment (start 161.455 99.13) (end 161.78001 99.45501) (width 0.25) (layer F.Cu) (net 12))
 (segment (start 161.455 98.255) (end 161.455 99.13) (width 0.25) (layer F.Cu) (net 12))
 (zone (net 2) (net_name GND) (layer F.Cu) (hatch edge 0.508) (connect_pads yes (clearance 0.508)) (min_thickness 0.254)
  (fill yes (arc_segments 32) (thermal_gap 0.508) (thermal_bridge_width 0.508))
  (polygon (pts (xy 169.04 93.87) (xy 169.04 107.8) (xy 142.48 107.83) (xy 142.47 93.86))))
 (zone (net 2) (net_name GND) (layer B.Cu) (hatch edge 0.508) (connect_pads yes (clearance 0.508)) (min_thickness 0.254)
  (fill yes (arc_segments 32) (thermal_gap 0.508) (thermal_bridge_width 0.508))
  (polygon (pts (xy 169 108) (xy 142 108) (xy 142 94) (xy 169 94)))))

